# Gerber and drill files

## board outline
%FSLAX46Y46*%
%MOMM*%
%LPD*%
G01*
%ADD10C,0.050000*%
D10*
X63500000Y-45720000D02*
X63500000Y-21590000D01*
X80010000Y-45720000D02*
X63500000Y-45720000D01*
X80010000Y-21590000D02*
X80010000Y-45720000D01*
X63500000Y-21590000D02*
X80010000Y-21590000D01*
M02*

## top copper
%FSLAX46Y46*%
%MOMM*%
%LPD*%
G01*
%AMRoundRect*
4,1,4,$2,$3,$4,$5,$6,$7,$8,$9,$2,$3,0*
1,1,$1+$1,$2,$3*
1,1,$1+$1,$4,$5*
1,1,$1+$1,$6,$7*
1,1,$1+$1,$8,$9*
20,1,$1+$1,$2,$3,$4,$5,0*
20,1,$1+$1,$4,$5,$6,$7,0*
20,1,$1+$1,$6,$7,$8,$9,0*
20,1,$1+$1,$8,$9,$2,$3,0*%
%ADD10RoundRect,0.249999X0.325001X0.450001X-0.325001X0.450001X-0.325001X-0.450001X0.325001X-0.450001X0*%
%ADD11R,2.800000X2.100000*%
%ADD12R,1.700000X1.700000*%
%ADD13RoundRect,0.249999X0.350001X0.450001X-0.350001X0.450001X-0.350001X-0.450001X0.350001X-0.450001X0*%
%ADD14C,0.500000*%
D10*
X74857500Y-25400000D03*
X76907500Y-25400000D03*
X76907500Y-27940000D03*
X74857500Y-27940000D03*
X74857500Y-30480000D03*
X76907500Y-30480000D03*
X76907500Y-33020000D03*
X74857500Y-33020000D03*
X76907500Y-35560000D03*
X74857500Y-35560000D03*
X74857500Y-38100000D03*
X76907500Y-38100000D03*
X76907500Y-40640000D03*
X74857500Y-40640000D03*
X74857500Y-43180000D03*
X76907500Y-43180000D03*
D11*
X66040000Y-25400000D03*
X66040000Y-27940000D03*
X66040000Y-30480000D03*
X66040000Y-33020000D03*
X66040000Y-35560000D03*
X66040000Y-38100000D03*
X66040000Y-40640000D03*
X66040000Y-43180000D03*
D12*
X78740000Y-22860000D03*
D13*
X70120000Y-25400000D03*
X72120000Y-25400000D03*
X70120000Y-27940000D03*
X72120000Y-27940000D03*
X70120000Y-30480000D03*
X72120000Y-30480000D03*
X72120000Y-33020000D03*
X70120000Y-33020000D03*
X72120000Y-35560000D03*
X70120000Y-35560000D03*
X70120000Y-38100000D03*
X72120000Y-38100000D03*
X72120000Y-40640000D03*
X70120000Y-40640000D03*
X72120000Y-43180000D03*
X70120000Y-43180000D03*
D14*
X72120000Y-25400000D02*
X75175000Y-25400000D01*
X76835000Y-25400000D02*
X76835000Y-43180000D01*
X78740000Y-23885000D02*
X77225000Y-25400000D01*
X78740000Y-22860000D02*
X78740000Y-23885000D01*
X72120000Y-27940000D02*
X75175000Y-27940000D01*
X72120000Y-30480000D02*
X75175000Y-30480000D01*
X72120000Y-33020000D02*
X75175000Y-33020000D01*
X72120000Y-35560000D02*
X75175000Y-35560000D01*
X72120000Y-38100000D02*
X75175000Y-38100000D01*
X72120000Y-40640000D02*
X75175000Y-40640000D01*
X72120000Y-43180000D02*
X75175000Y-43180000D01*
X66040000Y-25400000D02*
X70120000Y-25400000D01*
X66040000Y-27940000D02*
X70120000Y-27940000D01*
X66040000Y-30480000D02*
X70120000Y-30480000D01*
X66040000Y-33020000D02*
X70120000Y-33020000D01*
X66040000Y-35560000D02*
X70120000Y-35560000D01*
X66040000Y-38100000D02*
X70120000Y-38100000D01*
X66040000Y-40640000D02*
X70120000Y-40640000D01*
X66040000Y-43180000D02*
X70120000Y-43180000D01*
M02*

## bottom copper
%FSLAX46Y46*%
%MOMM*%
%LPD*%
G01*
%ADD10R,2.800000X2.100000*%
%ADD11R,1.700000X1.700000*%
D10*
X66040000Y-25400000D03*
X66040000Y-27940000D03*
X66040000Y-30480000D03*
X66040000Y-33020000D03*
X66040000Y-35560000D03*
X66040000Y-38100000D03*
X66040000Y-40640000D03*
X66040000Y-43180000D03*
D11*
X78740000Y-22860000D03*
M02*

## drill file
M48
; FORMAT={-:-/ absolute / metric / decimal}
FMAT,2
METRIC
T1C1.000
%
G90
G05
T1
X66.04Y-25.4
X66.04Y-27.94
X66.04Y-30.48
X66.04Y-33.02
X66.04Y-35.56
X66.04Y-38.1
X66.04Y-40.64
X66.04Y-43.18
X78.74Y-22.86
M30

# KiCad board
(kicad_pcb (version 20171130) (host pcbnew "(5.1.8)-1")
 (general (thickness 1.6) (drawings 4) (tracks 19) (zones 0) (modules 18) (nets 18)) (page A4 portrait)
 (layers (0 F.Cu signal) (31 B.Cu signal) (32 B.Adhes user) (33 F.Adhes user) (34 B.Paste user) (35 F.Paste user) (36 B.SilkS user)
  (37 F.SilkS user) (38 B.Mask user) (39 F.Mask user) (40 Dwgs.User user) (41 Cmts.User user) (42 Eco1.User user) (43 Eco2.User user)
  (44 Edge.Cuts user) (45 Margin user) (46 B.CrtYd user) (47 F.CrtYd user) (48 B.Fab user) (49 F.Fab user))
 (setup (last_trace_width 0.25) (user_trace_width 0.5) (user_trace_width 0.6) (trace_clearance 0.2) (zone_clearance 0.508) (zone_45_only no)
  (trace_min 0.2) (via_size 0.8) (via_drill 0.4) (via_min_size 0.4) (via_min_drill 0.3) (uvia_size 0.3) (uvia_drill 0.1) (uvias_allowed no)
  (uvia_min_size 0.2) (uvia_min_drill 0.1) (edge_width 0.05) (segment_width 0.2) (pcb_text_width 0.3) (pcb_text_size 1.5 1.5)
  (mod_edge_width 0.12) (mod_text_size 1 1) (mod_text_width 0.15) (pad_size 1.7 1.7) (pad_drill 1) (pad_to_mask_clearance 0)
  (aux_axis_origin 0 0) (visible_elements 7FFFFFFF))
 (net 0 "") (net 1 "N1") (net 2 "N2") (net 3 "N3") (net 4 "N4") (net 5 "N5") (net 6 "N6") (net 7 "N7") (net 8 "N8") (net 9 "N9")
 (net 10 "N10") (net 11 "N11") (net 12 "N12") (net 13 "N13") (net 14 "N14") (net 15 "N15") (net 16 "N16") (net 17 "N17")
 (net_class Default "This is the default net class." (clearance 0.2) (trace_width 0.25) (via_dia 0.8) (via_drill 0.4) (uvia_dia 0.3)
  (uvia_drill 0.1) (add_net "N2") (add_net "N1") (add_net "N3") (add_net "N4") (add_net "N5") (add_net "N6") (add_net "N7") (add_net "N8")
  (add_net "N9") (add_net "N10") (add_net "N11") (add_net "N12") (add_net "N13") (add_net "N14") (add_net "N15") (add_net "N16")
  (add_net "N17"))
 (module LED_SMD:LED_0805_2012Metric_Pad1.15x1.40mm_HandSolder (layer F.Cu) (at 75.8825 25.4 180)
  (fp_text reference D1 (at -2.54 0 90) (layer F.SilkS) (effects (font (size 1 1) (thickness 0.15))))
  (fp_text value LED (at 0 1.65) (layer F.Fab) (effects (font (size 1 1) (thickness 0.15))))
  (pad 2 smd roundrect (at 1.025 0 180) (size 1.15 1.4) (layers F.Cu F.Paste F.Mask) (roundrect_rratio 0.2173904347826087) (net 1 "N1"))
  (pad 1 smd roundrect (at -1.025 0 180) (size 1.15 1.4) (layers F.Cu F.Paste F.Mask) (roundrect_rratio 0.2173904347826087) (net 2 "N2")))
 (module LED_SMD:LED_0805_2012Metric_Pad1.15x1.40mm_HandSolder (layer F.Cu) (at 75.8825 27.94 180)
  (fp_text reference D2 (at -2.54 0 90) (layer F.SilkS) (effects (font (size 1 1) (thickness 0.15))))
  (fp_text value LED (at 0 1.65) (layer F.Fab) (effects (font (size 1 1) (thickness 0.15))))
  (pad 1 smd roundrect (at -1.025 0 180) (size 1.15 1.4) (layers F.Cu F.Paste F.Mask) (roundrect_rratio 0.2173904347826087) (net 2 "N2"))
  (pad 2 smd roundrect (at 1.025 0 180) (size 1.15 1.4) (layers F.Cu F.Paste F.Mask) (roundrect_rratio 0.2173904347826087) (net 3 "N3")))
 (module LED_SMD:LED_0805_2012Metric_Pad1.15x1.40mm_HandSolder (layer F.Cu) (at 75.8825 30.48 180)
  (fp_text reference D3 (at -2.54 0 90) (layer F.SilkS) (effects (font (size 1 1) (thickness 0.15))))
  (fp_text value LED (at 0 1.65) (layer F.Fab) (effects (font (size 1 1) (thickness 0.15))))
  (pad 2 smd roundrect (at 1.025 0 180) (size 1.15 1.4) (layers F.Cu F.Paste F.Mask) (roundrect_rratio 0.2173904347826087) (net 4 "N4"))
  (pad 1 smd roundrect (at -1.025 0 180) (size 1.15 1.4) (layers F.Cu F.Paste F.Mask) (roundrect_rratio 0.2173904347826087) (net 2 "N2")))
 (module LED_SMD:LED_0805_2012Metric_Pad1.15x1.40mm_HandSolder (layer F.Cu) (at 75.8825 33.02 180)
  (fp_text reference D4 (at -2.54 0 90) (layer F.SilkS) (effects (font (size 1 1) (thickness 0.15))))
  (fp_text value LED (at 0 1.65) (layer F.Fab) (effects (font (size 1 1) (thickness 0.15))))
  (pad 1 smd roundrect (at -1.025 0 180) (size 1.15 1.4) (layers F.Cu F.Paste F.Mask) (roundrect_rratio 0.2173904347826087) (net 2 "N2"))
  (pad 2 smd roundrect (at 1.025 0 180) (size 1.15 1.4) (layers F.Cu F.Paste F.Mask) (roundrect_rratio 0.2173904347826087) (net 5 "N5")))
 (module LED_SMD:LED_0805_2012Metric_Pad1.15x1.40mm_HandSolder (layer F.Cu) (at 75.8825 35.56 180)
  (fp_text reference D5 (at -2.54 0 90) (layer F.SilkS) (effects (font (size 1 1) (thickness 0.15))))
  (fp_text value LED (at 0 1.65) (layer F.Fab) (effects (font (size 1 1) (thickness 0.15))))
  (pad 1 smd roundrect (at -1.025 0 180) (size 1.15 1.4) (layers F.Cu F.Paste F.Mask) (roundrect_rratio 0.2173904347826087) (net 2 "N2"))
  (pad 2 smd roundrect (at 1.025 0 180) (size 1.15 1.4) (layers F.Cu F.Paste F.Mask) (roundrect_rratio 0.2173904347826087) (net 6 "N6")))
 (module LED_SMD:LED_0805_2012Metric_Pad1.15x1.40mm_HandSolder (layer F.Cu) (at 75.8825 38.1 180)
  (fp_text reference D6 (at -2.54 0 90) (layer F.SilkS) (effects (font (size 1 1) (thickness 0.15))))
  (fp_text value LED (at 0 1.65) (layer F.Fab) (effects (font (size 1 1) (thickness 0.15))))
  (pad 2 smd roundrect (at 1.025 0 180) (size 1.15 1.4) (layers F.Cu F.Paste F.Mask) (roundrect_rratio 0.2173904347826087) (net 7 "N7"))
  (pad 1 smd roundrect (at -1.025 0 180) (size 1.15 1.4) (layers F.Cu F.Paste F.Mask) (roundrect_rratio 0.2173904347826087) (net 2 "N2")))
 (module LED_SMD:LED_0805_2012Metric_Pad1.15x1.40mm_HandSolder (layer F.Cu) (at 75.8825 40.64 180)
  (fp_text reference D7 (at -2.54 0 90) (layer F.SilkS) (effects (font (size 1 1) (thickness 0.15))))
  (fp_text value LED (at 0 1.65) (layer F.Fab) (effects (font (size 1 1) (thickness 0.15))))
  (pad 1 smd roundrect (at -1.025 0 180) (size 1.15 1.4) (layers F.Cu F.Paste F.Mask) (roundrect_rratio 0.2173904347826087) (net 2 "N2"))
  (pad 2 smd roundrect (at 1.025 0 180) (size 1.15 1.4) (layers F.Cu F.Paste F.Mask) (roundrect_rratio 0.2173904347826087) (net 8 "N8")))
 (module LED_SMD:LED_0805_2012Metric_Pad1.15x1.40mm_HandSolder (layer F.Cu) (at 75.8825 43.18 180)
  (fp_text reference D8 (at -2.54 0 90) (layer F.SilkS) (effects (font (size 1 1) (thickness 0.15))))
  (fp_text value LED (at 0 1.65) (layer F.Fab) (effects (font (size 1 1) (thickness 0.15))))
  (pad 2 smd roundrect (at 1.025 0 180) (size 1.15 1.4) (layers F.Cu F.Paste F.Mask) (roundrect_rratio 0.2173904347826087) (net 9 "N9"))
  (pad 1 smd roundrect (at -1.025 0 180) (size 1.15 1.4) (layers F.Cu F.Paste F.Mask) (roundrect_rratio 0.2173904347826087) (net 2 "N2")))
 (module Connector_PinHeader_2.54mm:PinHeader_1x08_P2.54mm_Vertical (layer F.Cu) (at 66.04 25.4)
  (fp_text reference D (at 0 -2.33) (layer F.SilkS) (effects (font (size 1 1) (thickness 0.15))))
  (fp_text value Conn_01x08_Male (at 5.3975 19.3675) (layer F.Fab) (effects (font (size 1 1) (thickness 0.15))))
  (pad 1 thru_hole rect (at 0 0) (size 2.8 2.1) (drill 1) (layers *.Cu *.Mask) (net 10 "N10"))
  (pad 2 thru_hole rect (at 0 2.54) (size 2.8 2.1) (drill 1) (layers *.Cu *.Mask) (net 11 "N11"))
  (pad 3 thru_hole rect (at 0 5.08) (size 2.8 2.1) (drill 1) (layers *.Cu *.Mask) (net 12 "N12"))
  (pad 4 thru_hole rect (at 0 7.62) (size 2.8 2.1) (drill 1) (layers *.Cu *.Mask) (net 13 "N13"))
  (pad 5 thru_hole rect (at 0 10.16) (size 2.8 2.1) (drill 1) (layers *.Cu *.Mask) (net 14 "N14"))
  (pad 6 thru_hole rect (at 0 12.7) (size 2.8 2.1) (drill 1) (layers *.Cu *.Mask) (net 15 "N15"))
  (pad 7 thru_hole rect (at 0 15.24) (size 2.8 2.1) (drill 1) (layers *.Cu *.Mask) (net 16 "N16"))
  (pad 8 thru_hole rect (at 0 17.78) (size 2.8 2.1) (drill 1) (layers *.Cu *.Mask) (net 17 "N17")))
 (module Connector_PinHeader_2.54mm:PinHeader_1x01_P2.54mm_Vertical (layer F.Cu) (at 78.74 22.86)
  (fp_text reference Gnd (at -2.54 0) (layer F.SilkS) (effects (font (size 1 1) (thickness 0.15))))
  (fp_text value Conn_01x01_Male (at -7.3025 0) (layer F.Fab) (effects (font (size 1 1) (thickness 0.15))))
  (pad 1 thru_hole rect (at 0 0) (size 1.7 1.7) (drill 1) (layers *.Cu *.Mask) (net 2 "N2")))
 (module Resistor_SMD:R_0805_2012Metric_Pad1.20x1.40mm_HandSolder (layer F.Cu) (at 71.12 25.4 180)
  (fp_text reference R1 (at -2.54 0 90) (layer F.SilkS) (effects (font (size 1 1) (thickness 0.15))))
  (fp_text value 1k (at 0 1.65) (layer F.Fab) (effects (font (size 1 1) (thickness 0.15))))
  (pad 2 smd roundrect (at 1 0 180) (size 1.2 1.4) (layers F.Cu F.Paste F.Mask) (roundrect_rratio 0.2083325) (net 10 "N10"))
  (pad 1 smd roundrect (at -1 0 180) (size 1.2 1.4) (layers F.Cu F.Paste F.Mask) (roundrect_rratio 0.2083325) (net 1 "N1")))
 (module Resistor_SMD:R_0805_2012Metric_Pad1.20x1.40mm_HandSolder (layer F.Cu) (at 71.12 27.94 180)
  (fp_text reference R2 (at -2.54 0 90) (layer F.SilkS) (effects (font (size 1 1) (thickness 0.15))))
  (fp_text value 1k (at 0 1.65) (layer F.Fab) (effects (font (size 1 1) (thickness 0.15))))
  (pad 2 smd roundrect (at 1 0 180) (size 1.2 1.4) (layers F.Cu F.Paste F.Mask) (roundrect_rratio 0.2083325) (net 11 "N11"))
  (pad 1 smd roundrect (at -1 0 180) (size 1.2 1.4) (layers F.Cu F.Paste F.Mask) (roundrect_rratio 0.2083325) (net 3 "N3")))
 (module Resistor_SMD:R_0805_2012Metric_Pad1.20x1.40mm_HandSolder (layer F.Cu) (at 71.12 30.48 180)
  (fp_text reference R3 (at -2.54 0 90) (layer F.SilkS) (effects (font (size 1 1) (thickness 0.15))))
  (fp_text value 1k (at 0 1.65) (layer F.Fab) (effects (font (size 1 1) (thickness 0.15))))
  (pad 2 smd roundrect (at 1 0 180) (size 1.2 1.4) (layers F.Cu F.Paste F.Mask) (roundrect_rratio 0.2083325) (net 12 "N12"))
  (pad 1 smd roundrect (at -1 0 180) (size 1.2 1.4) (layers F.Cu F.Paste F.Mask) (roundrect_rratio 0.2083325) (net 4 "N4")))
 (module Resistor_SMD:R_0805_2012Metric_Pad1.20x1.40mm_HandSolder (layer F.Cu) (at 71.12 33.02 180)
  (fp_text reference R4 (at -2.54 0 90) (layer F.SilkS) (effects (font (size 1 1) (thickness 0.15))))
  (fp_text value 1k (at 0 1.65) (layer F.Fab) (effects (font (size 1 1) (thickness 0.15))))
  (pad 1 smd roundrect (at -1 0 180) (size 1.2 1.4) (layers F.Cu F.Paste F.Mask) (roundrect_rratio 0.2083325) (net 5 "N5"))
  (pad 2 smd roundrect (at 1 0 180) (size 1.2 1.4) (layers F.Cu F.Paste F.Mask) (roundrect_rratio 0.2083325) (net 13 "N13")))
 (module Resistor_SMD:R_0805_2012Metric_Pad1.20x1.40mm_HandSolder (layer F.Cu) (at 71.12 35.56 180)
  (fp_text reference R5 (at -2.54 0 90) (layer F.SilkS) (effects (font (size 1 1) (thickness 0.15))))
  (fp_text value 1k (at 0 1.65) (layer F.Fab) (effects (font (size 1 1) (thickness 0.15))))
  (pad 1 smd roundrect (at -1 0 180) (size 1.2 1.4) (layers F.Cu F.Paste F.Mask) (roundrect_rratio 0.2083325) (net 6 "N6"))
  (pad 2 smd roundrect (at 1 0 180) (size 1.2 1.4) (layers F.Cu F.Paste F.Mask) (roundrect_rratio 0.2083325) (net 14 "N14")))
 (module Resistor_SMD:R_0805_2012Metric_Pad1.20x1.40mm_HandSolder (layer F.Cu) (at 71.12 38.1 180)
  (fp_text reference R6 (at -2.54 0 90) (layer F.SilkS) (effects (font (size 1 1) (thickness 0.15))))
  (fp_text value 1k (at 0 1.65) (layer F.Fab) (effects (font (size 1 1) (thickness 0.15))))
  (pad 2 smd roundrect (at 1 0 180) (size 1.2 1.4) (layers F.Cu F.Paste F.Mask) (roundrect_rratio 0.2083325) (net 15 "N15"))
  (pad 1 smd roundrect (at -1 0 180) (size 1.2 1.4) (layers F.Cu F.Paste F.Mask) (roundrect_rratio 0.2083325) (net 7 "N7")))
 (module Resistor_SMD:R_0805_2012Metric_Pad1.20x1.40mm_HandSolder (layer F.Cu) (at 71.12 40.64 180)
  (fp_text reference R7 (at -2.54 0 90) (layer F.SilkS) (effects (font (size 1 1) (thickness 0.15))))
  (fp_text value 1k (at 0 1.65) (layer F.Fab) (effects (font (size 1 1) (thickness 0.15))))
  (pad 1 smd roundrect (at -1 0 180) (size 1.2 1.4) (layers F.Cu F.Paste F.Mask) (roundrect_rratio 0.2083325) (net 8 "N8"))
  (pad 2 smd roundrect (at 1 0 180) (size 1.2 1.4) (layers F.Cu F.Paste F.Mask) (roundrect_rratio 0.2083325) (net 16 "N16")))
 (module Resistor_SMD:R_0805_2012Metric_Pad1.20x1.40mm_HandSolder (layer F.Cu) (at 71.12 43.18 180)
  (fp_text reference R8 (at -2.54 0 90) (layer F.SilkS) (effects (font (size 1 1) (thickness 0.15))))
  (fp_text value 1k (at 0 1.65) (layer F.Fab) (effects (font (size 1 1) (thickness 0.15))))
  (pad 1 smd roundrect (at -1 0 180) (size 1.2 1.4) (layers F.Cu F.Paste F.Mask) (roundrect_rratio 0.2083325) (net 9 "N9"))
  (pad 2 smd roundrect (at 1 0 180) (size 1.2 1.4) (layers F.Cu F.Paste F.Mask) (roundrect_rratio 0.2083325) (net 17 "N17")))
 (gr_line (start 63.5 45.72) (end 63.5 21.59) (layer Edge.Cuts) (width 0.05))
 (gr_line (start 80.01 45.72) (end 63.5 45.72) (layer Edge.Cuts) (width 0.05))
 (gr_line (start 80.01 21.59) (end 80.01 45.72) (layer Edge.Cuts) (width 0.05))
 (gr_line (start 63.5 21.59) (end 80.01 21.59) (layer Edge.Cuts) (width 0.05))
 (segment (start 72.12 25.4) (end 75.175 25.4) (width 0.5) (layer F.Cu) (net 1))
 (segment (start 76.835 25.4) (end 76.835 43.18) (width 0.5) (layer F.Cu) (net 2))
 (segment (start 78.74 23.885) (end 77.225 25.4) (width 0.5) (layer F.Cu) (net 2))
 (segment (start 78.74 22.86) (end 78.74 23.885) (width 0.5) (layer F.Cu) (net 2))
 (segment (start 72.12 27.94) (end 75.175 27.94) (width 0.5) (layer F.Cu) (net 3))
 (segment (start 72.12 30.48) (end 75.175 30.48) (width 0.5) (layer F.Cu) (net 4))
 (segment (start 72.12 33.02) (end 75.175 33.02) (width 0.5) (layer F.Cu) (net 5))
 (segment (start 72.12 35.56) (end 75.175 35.56) (width 0.5) (layer F.Cu) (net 6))
 (segment (start 72.12 38.1) (end 75.175 38.1) (width 0.5) (layer F.Cu) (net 7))
 (segment (start 72.12 40.64) (end 75.175 40.64) (width 0.5) (layer F.Cu) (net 8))
 (segment (start 72.12 43.18) (end 75.175 43.18) (width 0.5) (layer F.Cu) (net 9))
 (segment (start 66.04 25.4) (end 70.12 25.4) (width 0.5) (layer F.Cu) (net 10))
 (segment (start 66.04 27.94) (end 70.12 27.94) (width 0.5) (layer F.Cu) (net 11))
 (segment (start 66.04 30.48) (end 70.12 30.48) (width 0.5) (layer F.Cu) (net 12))
 (segment (start 66.04 33.02) (end 70.12 33.02) (width 0.5) (layer F.Cu) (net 13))
 (segment (start 66.04 35.56) (end 70.12 35.56) (width 0.5) (layer F.Cu) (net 14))
 (segment (start 66.04 38.1) (end 70.12 38.1) (width 0.5) (layer F.Cu) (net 15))
 (segment (start 66.04 40.64) (end 70.12 40.64) (width 0.5) (layer F.Cu) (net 16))
 (segment (start 66.04 43.18) (end 70.12 43.18) (width 0.5) (layer F.Cu) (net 17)))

